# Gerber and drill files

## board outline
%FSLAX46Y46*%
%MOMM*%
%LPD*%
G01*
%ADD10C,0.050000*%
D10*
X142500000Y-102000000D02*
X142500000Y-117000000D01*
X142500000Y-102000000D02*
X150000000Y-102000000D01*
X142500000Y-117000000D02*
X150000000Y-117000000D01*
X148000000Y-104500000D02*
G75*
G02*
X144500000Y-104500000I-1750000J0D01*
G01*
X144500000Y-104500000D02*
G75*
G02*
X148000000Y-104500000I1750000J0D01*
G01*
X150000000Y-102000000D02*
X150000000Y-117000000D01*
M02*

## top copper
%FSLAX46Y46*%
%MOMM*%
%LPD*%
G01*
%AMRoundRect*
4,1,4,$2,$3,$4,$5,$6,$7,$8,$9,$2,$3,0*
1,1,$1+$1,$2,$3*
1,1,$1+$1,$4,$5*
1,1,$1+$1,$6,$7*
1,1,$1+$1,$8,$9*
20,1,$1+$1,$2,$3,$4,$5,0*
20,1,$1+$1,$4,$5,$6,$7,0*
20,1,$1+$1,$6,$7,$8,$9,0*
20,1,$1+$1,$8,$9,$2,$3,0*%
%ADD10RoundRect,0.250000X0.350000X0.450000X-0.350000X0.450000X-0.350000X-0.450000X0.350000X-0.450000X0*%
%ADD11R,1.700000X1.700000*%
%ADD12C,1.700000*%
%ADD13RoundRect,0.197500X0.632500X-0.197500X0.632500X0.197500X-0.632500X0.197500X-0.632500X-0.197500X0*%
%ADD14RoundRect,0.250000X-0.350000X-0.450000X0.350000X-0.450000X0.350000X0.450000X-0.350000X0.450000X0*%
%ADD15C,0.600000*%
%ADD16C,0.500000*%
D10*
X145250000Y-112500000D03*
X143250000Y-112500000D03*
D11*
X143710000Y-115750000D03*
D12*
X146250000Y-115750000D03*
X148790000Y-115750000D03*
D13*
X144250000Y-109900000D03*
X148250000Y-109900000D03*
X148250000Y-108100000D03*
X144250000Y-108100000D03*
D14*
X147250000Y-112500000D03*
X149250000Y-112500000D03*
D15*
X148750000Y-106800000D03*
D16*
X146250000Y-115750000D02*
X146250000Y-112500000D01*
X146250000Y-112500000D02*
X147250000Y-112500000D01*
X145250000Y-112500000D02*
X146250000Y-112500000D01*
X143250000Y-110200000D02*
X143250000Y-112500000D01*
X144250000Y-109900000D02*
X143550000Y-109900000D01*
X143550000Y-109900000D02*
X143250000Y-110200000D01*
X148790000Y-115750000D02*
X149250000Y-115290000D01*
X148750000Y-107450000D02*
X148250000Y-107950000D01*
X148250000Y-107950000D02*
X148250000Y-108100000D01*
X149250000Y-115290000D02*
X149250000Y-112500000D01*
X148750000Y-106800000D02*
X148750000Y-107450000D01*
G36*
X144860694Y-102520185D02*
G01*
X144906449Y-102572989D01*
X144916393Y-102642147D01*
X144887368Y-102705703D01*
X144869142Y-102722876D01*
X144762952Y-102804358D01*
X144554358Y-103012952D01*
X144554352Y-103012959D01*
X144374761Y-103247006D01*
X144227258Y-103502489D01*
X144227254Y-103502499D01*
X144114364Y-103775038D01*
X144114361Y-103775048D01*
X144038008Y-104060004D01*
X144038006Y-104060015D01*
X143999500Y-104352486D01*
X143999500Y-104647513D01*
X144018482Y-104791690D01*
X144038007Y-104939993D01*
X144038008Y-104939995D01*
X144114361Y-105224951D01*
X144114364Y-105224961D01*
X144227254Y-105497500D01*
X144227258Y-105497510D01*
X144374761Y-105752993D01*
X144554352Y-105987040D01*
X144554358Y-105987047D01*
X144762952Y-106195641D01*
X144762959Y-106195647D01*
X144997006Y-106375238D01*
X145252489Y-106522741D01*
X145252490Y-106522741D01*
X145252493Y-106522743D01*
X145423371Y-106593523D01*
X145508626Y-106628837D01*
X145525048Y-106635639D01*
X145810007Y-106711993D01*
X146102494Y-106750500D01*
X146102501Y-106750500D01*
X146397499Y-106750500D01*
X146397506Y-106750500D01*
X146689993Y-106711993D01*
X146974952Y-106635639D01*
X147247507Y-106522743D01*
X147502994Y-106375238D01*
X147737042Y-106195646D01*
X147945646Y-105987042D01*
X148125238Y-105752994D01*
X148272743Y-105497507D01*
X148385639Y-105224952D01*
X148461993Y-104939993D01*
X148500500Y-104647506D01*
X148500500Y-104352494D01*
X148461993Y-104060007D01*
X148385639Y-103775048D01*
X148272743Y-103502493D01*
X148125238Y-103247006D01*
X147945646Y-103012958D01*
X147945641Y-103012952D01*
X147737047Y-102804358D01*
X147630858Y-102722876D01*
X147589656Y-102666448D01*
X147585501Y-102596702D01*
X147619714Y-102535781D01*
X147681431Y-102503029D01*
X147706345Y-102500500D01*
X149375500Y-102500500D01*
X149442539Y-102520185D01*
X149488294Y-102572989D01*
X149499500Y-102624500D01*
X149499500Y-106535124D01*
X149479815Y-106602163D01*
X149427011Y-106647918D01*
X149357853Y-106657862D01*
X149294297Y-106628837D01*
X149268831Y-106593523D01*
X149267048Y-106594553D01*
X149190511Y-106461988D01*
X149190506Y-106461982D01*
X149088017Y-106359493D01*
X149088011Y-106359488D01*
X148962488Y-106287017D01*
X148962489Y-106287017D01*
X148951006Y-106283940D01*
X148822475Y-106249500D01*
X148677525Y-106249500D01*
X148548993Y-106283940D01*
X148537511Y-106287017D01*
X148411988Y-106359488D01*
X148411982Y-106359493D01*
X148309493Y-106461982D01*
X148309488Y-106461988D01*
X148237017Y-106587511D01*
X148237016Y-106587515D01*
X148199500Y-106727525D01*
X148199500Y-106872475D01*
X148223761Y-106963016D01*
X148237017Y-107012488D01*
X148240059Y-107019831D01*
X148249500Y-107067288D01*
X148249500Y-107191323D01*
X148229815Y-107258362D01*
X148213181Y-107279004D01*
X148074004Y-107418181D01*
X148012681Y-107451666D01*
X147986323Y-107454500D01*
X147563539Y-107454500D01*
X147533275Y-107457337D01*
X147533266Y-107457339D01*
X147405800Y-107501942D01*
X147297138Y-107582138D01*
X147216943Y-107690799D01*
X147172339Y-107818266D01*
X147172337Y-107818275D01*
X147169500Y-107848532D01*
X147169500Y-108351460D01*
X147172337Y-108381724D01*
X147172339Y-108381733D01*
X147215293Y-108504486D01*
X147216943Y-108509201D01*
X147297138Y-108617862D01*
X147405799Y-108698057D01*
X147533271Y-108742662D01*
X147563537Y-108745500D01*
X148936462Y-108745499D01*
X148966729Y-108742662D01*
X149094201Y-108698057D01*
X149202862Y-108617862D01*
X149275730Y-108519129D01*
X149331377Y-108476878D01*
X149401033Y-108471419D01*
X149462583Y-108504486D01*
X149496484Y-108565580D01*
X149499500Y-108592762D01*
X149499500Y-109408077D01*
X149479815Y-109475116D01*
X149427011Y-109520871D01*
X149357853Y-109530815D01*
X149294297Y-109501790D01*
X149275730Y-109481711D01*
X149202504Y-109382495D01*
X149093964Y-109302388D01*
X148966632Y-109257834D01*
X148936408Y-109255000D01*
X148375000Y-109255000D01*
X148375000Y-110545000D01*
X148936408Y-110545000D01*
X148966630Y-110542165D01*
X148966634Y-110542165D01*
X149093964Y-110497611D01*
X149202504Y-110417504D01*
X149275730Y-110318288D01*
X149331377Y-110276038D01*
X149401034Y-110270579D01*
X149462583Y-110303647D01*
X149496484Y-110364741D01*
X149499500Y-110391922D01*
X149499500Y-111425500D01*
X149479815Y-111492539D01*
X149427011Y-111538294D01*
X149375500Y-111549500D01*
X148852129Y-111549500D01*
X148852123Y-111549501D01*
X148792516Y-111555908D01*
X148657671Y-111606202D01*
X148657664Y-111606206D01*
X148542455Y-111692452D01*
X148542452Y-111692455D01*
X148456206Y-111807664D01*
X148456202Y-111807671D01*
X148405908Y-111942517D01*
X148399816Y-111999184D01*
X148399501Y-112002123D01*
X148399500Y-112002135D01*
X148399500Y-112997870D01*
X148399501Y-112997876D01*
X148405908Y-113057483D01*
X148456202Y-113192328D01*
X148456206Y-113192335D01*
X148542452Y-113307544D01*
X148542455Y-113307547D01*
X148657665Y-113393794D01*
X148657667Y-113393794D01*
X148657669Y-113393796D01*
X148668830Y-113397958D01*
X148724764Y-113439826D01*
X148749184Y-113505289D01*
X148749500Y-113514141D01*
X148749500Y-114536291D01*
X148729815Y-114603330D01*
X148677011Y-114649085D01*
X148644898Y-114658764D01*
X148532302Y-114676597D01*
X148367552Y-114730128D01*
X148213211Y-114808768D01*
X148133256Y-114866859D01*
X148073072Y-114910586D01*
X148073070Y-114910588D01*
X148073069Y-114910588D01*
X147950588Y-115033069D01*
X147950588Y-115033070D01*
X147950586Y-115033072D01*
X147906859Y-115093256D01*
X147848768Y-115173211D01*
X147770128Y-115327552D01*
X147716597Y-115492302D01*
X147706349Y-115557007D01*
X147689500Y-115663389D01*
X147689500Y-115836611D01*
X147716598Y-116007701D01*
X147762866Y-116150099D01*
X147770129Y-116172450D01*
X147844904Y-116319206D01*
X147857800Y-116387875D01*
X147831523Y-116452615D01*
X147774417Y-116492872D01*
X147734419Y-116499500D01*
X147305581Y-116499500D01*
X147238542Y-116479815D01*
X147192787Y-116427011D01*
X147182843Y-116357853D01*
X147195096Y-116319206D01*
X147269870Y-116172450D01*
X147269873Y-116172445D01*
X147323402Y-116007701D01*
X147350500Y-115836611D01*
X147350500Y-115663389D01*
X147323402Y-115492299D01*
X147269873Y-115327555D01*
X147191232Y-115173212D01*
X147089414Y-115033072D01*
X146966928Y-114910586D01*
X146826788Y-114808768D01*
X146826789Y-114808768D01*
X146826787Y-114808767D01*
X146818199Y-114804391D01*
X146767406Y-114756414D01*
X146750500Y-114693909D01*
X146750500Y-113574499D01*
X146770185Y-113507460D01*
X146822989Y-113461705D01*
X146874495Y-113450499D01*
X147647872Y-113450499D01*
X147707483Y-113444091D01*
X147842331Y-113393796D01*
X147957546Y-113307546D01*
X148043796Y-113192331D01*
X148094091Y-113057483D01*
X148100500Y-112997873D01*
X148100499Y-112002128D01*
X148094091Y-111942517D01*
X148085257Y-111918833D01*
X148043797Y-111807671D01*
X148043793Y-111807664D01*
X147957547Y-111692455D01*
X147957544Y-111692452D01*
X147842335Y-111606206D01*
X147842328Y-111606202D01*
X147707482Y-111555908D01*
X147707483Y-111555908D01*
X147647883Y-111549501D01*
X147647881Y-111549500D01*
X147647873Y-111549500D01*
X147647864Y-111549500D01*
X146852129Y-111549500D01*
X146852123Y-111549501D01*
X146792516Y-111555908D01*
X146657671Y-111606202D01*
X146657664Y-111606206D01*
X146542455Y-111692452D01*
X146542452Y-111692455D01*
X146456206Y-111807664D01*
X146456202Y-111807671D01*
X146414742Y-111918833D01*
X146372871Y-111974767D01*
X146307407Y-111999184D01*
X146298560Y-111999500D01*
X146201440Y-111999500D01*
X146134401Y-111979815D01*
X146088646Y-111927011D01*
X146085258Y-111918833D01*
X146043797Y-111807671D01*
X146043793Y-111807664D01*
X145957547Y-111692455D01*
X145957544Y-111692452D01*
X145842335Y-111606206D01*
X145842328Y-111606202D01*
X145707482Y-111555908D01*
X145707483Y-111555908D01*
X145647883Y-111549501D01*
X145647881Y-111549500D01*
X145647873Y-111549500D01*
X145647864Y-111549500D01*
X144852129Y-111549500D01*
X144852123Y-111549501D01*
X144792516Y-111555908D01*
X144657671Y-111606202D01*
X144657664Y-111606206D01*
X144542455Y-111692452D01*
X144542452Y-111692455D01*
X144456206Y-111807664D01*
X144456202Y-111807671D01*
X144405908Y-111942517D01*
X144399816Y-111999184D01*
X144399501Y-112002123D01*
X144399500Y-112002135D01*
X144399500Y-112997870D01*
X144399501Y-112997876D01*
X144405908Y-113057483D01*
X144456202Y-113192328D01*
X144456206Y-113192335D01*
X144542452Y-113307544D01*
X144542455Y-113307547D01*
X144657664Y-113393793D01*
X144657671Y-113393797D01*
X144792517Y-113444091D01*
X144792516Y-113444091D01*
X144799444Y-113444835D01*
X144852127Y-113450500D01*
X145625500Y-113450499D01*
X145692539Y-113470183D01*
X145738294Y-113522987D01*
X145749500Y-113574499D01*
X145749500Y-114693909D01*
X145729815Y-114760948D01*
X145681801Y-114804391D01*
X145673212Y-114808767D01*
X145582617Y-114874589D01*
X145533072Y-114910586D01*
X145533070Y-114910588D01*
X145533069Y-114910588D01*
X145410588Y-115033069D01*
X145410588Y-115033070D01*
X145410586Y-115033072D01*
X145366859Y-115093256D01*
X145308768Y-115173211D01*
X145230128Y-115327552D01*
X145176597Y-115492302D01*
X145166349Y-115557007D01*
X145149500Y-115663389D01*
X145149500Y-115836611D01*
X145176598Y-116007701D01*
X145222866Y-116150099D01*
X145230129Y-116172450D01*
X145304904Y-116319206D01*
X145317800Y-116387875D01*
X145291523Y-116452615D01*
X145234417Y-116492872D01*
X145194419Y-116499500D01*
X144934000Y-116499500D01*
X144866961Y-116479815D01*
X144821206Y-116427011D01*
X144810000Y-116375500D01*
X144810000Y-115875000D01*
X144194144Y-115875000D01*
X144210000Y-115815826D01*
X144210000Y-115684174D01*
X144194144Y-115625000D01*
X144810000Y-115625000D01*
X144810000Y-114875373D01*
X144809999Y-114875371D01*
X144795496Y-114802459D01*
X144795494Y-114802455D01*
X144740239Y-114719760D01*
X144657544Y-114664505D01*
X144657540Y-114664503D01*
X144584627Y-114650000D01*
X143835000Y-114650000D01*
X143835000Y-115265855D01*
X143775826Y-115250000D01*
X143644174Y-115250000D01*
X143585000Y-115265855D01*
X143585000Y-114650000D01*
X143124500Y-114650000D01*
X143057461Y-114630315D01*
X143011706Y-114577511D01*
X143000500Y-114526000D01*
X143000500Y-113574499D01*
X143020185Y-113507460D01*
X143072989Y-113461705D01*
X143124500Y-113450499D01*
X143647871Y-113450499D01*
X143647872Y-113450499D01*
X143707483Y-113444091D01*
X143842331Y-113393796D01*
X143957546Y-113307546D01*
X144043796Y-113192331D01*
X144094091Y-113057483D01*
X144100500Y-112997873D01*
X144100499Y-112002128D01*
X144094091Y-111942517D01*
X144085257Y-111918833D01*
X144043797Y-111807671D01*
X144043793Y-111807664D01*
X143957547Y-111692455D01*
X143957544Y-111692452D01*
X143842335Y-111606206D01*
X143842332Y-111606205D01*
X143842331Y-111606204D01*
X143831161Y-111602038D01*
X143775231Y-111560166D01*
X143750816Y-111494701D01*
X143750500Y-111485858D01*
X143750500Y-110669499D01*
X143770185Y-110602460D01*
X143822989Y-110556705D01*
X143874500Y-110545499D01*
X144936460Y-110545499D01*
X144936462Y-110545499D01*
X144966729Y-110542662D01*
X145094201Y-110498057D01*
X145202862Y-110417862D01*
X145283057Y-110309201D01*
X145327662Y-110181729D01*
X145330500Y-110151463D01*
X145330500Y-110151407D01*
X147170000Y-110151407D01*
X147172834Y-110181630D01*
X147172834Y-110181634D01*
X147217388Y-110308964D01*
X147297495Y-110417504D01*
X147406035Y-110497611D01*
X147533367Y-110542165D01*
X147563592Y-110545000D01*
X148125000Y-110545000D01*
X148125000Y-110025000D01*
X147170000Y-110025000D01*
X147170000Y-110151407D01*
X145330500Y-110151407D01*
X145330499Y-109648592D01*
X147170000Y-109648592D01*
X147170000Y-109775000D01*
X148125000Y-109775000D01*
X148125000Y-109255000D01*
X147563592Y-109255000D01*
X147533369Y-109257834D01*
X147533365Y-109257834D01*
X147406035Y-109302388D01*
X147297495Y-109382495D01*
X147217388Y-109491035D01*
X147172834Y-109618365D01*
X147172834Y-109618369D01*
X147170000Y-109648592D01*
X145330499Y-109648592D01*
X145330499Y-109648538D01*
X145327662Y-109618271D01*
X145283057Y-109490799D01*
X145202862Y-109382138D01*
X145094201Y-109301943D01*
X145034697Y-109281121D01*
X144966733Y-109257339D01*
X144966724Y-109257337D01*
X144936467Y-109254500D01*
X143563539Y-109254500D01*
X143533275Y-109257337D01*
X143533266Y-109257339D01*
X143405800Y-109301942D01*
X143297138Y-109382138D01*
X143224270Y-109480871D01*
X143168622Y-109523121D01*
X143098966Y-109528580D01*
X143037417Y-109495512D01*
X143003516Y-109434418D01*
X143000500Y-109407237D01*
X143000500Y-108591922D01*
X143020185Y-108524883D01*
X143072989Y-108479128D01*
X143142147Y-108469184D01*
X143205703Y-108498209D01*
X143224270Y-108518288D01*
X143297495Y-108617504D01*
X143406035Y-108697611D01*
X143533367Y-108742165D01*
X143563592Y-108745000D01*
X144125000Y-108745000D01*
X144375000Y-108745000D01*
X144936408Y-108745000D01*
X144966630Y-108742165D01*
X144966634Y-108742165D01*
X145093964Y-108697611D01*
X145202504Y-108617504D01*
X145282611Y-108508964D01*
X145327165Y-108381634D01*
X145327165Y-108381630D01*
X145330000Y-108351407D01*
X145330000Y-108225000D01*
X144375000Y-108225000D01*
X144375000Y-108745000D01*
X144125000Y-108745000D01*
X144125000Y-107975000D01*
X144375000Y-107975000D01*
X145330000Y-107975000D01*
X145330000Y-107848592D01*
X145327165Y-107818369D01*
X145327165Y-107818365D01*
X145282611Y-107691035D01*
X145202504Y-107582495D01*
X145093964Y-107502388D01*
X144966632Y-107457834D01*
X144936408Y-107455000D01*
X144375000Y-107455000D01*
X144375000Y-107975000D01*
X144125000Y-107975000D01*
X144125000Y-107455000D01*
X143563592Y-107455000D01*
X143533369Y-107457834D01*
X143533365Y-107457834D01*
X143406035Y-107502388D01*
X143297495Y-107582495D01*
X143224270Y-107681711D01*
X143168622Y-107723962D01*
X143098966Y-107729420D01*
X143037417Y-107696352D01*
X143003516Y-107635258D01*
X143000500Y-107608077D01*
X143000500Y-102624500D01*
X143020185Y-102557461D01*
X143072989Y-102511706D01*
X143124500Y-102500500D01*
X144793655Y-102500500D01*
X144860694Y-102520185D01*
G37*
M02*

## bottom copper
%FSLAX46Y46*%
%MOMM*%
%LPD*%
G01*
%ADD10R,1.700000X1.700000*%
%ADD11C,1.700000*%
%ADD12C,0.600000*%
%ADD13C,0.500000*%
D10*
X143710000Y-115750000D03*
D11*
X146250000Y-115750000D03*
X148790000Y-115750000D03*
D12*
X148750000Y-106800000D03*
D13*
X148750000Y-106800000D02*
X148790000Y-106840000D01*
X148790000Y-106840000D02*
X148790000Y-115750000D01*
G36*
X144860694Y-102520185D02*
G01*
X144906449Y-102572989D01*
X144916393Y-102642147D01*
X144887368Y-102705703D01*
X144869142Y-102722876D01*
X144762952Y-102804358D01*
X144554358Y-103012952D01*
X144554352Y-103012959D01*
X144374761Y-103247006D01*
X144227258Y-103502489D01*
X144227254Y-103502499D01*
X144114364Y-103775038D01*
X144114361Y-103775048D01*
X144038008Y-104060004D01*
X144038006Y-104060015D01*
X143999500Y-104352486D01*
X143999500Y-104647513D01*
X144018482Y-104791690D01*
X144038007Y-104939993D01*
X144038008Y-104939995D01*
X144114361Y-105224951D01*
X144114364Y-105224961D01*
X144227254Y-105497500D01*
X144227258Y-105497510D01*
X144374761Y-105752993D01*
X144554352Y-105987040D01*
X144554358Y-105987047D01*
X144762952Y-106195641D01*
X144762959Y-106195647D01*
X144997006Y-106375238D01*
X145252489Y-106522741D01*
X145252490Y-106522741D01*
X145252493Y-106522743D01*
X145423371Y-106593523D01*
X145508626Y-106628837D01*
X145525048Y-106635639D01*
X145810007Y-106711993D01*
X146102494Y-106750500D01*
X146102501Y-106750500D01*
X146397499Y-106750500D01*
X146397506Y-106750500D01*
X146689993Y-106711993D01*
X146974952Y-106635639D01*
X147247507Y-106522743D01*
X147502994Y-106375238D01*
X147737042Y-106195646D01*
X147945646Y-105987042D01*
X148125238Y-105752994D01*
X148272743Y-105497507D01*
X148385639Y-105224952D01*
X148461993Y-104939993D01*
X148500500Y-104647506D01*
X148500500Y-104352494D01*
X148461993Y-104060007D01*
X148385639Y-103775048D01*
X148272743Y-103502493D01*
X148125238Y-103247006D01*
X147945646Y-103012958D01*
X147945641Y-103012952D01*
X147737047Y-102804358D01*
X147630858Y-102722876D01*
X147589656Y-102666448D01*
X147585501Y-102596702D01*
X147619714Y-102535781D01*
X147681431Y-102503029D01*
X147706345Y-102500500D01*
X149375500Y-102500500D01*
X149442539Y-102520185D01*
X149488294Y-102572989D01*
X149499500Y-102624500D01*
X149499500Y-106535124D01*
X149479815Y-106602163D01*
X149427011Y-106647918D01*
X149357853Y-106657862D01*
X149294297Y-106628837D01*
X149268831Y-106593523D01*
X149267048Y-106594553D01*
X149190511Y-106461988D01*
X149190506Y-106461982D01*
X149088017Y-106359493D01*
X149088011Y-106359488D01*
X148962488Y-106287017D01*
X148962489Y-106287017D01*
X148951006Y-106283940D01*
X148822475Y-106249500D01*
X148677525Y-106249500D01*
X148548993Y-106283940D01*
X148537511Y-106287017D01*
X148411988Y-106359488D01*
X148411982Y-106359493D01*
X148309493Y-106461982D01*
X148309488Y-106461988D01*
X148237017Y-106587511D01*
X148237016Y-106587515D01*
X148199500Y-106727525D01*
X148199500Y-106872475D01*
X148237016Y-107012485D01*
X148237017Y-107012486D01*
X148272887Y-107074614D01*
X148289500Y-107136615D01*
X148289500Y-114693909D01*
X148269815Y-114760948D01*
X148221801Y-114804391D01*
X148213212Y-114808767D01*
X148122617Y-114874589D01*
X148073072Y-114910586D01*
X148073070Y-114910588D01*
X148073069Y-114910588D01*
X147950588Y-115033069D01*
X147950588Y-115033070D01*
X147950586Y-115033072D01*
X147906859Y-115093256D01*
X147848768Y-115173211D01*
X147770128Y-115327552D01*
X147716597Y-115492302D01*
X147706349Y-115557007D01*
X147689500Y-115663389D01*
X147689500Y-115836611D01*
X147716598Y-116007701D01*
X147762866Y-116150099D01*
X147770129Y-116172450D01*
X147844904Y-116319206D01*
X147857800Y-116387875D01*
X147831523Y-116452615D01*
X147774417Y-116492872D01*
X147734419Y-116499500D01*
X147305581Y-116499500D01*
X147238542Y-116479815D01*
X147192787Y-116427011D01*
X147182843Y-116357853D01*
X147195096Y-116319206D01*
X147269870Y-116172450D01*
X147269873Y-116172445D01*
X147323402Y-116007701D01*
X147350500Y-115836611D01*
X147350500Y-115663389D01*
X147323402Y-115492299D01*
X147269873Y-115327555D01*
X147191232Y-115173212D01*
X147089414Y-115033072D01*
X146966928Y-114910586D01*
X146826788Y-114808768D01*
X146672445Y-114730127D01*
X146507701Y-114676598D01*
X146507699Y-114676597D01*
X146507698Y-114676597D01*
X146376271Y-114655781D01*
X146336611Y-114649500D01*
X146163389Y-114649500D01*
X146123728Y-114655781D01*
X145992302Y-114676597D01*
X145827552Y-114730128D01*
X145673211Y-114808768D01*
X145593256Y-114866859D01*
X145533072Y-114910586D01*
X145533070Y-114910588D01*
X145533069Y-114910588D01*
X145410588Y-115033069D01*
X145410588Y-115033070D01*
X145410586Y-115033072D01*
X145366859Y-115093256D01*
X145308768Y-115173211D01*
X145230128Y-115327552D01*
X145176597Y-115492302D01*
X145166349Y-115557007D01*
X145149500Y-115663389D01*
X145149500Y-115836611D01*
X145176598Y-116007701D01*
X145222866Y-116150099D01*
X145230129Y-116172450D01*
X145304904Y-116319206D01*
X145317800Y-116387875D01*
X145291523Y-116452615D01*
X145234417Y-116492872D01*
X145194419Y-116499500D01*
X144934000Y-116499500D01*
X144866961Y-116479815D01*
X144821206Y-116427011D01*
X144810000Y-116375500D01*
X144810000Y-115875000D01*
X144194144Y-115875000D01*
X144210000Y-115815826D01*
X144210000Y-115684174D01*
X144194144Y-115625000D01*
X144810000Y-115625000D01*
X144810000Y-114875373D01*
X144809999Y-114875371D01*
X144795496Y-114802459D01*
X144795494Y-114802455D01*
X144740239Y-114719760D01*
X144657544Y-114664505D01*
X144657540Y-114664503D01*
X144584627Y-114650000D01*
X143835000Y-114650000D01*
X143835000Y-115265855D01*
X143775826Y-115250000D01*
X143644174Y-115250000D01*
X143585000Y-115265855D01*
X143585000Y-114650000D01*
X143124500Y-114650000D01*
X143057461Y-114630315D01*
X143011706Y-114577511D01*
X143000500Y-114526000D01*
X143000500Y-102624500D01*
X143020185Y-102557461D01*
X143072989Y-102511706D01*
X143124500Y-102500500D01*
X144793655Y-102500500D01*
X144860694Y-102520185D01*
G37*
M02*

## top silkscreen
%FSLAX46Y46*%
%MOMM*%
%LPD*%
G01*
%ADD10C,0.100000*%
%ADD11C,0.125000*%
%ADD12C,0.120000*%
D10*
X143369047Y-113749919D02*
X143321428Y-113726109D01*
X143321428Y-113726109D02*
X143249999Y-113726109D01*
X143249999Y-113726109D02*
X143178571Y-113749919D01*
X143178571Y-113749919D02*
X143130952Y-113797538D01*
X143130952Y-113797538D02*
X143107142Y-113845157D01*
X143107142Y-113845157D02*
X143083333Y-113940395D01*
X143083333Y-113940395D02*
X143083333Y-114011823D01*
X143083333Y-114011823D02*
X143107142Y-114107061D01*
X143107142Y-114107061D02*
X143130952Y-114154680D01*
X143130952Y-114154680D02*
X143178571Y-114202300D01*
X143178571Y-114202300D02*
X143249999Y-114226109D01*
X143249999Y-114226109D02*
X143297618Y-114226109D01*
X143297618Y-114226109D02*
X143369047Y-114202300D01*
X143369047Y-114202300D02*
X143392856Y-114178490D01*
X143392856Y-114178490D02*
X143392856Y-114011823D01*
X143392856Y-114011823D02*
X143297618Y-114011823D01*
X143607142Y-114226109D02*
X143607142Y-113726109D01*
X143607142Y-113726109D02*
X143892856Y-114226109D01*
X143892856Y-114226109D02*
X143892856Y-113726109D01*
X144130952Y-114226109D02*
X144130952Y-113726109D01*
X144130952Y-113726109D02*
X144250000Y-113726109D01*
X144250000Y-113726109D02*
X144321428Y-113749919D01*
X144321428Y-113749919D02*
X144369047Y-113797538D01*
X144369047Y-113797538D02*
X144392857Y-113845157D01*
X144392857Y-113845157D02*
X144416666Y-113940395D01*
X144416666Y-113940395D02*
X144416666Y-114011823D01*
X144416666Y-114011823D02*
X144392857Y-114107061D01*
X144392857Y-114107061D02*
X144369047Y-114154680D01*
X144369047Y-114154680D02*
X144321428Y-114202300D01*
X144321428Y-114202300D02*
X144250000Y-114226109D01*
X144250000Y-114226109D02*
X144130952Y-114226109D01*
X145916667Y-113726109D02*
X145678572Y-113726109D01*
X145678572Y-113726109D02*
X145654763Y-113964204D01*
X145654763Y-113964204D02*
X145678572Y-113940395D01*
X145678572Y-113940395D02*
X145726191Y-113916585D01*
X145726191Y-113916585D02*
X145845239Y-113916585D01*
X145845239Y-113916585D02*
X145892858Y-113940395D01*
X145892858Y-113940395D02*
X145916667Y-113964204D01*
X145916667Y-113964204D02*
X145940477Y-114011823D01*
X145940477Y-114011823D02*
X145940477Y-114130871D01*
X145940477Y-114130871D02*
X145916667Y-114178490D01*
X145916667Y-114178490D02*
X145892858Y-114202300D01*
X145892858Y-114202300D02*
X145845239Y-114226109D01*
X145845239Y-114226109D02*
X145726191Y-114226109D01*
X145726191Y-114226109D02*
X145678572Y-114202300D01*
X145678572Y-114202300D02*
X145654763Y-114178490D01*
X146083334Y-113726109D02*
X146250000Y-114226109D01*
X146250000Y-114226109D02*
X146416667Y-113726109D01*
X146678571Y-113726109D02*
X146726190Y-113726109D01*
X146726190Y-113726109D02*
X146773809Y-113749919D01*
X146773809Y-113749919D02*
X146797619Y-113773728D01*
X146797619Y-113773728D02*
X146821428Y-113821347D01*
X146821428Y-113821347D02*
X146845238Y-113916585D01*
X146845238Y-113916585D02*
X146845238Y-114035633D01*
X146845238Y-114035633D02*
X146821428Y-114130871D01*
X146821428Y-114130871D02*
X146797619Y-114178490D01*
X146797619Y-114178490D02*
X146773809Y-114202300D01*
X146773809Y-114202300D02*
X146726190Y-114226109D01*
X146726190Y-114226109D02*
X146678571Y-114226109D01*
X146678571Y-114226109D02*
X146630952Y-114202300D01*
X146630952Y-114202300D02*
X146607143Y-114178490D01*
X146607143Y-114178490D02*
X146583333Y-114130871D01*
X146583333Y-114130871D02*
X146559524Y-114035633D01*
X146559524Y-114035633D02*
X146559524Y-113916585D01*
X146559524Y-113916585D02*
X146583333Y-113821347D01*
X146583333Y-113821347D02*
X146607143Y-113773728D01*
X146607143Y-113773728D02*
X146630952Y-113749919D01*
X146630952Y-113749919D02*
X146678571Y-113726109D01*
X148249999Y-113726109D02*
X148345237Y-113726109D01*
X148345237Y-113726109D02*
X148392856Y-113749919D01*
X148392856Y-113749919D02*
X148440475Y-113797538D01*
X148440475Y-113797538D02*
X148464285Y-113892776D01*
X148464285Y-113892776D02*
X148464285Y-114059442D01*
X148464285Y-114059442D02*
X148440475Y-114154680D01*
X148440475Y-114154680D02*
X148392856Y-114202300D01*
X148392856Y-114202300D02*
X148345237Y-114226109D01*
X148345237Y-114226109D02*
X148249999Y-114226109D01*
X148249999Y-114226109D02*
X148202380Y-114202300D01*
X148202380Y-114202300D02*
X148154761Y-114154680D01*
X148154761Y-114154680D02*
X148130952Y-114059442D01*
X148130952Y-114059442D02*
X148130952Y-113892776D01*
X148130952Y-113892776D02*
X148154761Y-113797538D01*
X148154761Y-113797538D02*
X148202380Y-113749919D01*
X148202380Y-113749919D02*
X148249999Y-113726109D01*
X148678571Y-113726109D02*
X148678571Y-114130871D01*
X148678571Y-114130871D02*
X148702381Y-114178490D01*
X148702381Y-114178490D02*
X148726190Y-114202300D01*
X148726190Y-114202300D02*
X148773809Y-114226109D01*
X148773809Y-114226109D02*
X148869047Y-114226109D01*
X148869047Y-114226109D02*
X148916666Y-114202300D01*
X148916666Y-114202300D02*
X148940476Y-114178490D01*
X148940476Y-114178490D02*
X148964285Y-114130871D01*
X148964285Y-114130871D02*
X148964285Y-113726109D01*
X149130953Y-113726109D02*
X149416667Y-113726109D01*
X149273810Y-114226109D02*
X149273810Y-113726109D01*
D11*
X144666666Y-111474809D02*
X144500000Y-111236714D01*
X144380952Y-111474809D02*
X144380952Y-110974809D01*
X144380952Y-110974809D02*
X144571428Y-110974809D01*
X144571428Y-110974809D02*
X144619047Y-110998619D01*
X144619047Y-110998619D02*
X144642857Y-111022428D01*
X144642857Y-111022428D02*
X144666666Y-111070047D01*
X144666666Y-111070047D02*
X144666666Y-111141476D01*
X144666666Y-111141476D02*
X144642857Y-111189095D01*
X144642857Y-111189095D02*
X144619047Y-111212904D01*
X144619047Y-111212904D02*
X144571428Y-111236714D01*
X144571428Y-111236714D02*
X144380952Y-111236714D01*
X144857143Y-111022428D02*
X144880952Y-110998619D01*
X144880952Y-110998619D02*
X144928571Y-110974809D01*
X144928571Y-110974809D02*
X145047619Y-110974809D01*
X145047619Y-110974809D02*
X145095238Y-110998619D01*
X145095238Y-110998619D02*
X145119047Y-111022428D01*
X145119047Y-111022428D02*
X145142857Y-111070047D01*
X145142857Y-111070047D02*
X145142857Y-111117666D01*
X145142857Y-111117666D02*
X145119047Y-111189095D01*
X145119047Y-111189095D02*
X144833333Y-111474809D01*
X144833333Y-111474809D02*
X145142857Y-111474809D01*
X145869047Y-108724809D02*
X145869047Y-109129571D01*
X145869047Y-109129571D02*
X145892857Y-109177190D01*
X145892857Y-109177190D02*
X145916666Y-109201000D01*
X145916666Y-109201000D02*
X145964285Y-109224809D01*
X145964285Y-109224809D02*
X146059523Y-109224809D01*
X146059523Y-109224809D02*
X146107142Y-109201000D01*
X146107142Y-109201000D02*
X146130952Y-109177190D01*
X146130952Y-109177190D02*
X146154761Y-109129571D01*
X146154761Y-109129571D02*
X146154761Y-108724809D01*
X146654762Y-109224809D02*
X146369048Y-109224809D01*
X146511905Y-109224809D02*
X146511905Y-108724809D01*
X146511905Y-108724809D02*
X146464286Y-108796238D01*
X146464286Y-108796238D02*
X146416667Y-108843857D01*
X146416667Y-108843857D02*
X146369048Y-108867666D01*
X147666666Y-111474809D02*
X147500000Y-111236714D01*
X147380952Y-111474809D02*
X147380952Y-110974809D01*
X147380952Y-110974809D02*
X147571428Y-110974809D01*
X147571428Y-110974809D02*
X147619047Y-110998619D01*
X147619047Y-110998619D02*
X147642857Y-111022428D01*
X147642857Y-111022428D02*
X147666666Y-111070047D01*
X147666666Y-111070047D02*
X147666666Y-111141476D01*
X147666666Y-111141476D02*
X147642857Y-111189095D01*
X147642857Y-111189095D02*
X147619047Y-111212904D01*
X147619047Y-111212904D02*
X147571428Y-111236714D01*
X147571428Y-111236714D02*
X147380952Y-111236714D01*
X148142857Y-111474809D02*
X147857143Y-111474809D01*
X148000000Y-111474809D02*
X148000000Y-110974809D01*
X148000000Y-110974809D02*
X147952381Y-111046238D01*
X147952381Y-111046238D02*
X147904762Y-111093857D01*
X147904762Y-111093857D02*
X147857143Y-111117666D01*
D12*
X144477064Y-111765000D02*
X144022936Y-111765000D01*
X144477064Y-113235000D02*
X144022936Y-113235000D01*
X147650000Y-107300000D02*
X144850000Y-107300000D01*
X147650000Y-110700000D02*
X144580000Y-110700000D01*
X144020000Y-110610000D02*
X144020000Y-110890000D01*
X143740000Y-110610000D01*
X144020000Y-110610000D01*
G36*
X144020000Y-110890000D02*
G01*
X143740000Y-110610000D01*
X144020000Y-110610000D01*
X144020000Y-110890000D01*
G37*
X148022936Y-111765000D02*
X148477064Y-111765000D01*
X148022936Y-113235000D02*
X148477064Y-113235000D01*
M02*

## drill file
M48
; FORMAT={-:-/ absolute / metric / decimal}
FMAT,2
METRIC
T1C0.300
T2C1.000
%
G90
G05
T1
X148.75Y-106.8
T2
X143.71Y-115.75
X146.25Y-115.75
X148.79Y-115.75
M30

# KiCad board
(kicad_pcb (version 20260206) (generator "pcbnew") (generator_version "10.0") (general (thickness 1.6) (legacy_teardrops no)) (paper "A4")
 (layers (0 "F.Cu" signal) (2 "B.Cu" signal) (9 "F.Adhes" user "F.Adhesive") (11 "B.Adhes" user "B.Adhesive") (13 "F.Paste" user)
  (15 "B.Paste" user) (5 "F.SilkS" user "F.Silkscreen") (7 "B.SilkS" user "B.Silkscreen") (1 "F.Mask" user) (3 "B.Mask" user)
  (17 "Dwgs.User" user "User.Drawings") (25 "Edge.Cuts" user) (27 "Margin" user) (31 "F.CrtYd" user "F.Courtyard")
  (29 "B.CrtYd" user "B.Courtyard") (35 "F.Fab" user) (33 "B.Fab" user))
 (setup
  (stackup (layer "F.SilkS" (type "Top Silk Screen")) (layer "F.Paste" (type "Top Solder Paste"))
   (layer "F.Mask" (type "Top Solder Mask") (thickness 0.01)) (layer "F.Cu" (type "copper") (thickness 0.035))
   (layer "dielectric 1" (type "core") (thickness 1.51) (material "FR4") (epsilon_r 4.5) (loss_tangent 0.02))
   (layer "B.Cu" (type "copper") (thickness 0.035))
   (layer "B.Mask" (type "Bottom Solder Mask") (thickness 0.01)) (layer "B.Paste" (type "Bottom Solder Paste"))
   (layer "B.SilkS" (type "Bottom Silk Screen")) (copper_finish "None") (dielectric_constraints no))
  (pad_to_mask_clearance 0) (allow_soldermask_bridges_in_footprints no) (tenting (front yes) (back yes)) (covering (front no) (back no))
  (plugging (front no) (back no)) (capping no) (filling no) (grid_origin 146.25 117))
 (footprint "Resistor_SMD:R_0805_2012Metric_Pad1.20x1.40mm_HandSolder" (layer "F.Cu") (at 144.25 112.5 180)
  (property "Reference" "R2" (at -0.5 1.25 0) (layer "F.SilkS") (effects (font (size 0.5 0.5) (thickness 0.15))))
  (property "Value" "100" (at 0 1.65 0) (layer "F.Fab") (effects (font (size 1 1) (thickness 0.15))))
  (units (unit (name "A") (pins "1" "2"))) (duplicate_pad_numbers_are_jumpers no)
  (fp_line (start -0.227064 0.735) (end 0.227064 0.735) (stroke (width 0.12) (type solid)) (layer "F.SilkS"))
  (fp_line (start -0.227064 -0.735) (end 0.227064 -0.735) (stroke (width 0.12) (type solid)) (layer "F.SilkS"))
  (pad "1" smd roundrect (at -1 0 180) (size 1.2 1.4) (layers "F.Cu" "F.Mask" "F.Paste") (roundrect_rratio 0.208333) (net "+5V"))
  (pad "2" smd roundrect (at 1 0 180) (size 1.2 1.4) (layers "F.Cu" "F.Mask" "F.Paste") (roundrect_rratio 0.208333) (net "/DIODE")))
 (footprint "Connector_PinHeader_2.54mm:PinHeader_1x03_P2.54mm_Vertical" (layer "F.Cu") (at 143.71 115.75 90)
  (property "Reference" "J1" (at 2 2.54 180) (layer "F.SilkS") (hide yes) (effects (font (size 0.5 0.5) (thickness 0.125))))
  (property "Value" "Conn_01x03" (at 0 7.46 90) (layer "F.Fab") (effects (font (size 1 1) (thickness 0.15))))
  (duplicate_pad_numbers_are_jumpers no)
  (pad "1" thru_hole rect (at 0 0 90) (size 1.7 1.7) (drill 1) (layers "*.Cu" "*.Mask") (remove_unused_layers no) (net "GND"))
  (pad "2" thru_hole circle (at 0 2.54 90) (size 1.7 1.7) (drill 1) (layers "*.Cu" "*.Mask") (remove_unused_layers no) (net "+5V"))
  (pad "3" thru_hole circle (at 0 5.08 90) (size 1.7 1.7) (drill 1) (layers "*.Cu" "*.Mask") (remove_unused_layers no) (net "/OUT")))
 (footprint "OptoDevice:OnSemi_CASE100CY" (layer "F.Cu") (at 146.25 109 90)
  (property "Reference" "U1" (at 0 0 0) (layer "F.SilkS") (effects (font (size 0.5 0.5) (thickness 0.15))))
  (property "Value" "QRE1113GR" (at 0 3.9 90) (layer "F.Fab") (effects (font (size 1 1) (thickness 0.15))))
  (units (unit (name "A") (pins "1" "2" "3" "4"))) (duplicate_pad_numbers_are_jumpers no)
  (fp_line (start 1.7 1.4) (end 1.7 -1.4) (stroke (width 0.12) (type solid)) (layer "F.SilkS"))
  (fp_line (start -1.7 1.4) (end -1.7 -1.67) (stroke (width 0.12) (type solid)) (layer "F.SilkS"))
  (fp_poly
   (pts (xy -1.61 -2.23) (xy -1.89 -2.23) (xy -1.61 -2.51) (xy -1.61 -2.23)) (stroke (width 0.12) (type solid)) (fill yes) (layer "F.SilkS"))
  (pad "1" smd roundrect (at -0.9 -2 90) (size 0.79 1.66) (layers "F.Cu" "F.Mask" "F.Paste") (roundrect_rratio 0.25) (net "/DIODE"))
  (pad "2" smd roundrect (at -0.9 2 90) (size 0.79 1.66) (layers "F.Cu" "F.Mask" "F.Paste") (roundrect_rratio 0.25) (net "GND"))
  (pad "3" smd roundrect (at 0.9 2 90) (size 0.79 1.66) (layers "F.Cu" "F.Mask" "F.Paste") (roundrect_rratio 0.25) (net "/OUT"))
  (pad "4" smd roundrect (at 0.9 -2 90) (size 0.79 1.66) (layers "F.Cu" "F.Mask" "F.Paste") (roundrect_rratio 0.25) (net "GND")))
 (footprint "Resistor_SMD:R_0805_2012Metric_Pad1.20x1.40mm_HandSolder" (layer "F.Cu") (at 148.25 112.5)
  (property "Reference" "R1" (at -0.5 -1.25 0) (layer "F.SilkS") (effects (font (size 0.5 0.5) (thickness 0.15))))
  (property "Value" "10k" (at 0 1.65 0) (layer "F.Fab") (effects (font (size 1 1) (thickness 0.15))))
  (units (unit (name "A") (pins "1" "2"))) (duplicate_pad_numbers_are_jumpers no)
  (fp_line (start -0.227064 -0.735) (end 0.227064 -0.735) (stroke (width 0.12) (type solid)) (layer "F.SilkS"))
  (fp_line (start -0.227064 0.735) (end 0.227064 0.735) (stroke (width 0.12) (type solid)) (layer "F.SilkS"))
  (pad "1" smd roundrect (at -1 0) (size 1.2 1.4) (layers "F.Cu" "F.Mask" "F.Paste") (roundrect_rratio 0.208333) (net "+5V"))
  (pad "2" smd roundrect (at 1 0) (size 1.2 1.4) (layers "F.Cu" "F.Mask" "F.Paste") (roundrect_rratio 0.208333) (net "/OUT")))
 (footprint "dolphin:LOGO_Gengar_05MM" (layer "B.Cu") (at 146.25 109 180)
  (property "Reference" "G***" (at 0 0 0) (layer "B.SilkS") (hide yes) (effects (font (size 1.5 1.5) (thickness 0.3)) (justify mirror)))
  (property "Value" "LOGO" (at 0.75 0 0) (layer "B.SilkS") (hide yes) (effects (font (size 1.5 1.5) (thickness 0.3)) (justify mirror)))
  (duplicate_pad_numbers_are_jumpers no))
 (gr_line (start 142.5 102) (end 142.5 117) (stroke (width 0.05) (type default)) (layer "Edge.Cuts"))
 (gr_line (start 142.5 102) (end 150 102) (stroke (width 0.05) (type default)) (layer "Edge.Cuts"))
 (gr_line (start 142.5 117) (end 150 117) (stroke (width 0.05) (type default)) (layer "Edge.Cuts"))
 (gr_circle (center 146.25 104.5) (end 148 104.5) (stroke (width 0.05) (type default)) (fill no) (layer "Edge.Cuts"))
 (gr_line (start 150 102) (end 150 117) (stroke (width 0.05) (type default)) (layer "Edge.Cuts"))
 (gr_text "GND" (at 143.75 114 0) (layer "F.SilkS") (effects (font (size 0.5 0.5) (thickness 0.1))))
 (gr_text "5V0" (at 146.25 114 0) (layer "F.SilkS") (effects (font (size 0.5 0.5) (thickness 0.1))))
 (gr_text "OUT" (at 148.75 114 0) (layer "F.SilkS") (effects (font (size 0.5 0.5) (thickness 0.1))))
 (segment (start 146.25 115.75) (end 146.25 112.5) (width 0.5) (layer "F.Cu") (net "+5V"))
 (segment (start 146.25 112.5) (end 147.25 112.5) (width 0.5) (layer "F.Cu") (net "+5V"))
 (segment (start 145.25 112.5) (end 146.25 112.5) (width 0.5) (layer "F.Cu") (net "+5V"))
 (segment (start 143.25 110.2) (end 143.25 112.5) (width 0.5) (layer "F.Cu") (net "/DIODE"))
 (segment (start 144.25 109.9) (end 143.55 109.9) (width 0.5) (layer "F.Cu") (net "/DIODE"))
 (segment (start 143.55 109.9) (end 143.25 110.2) (width 0.5) (layer "F.Cu") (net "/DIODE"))
 (segment (start 148.79 115.75) (end 149.25 115.29) (width 0.5) (layer "F.Cu") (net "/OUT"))
 (segment (start 148.75 107.45) (end 148.25 107.95) (width 0.5) (layer "F.Cu") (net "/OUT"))
 (segment (start 148.25 107.95) (end 148.25 108.1) (width 0.5) (layer "F.Cu") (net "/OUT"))
 (segment (start 149.25 115.29) (end 149.25 112.5) (width 0.5) (layer "F.Cu") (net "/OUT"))
 (segment (start 148.75 106.8) (end 148.75 107.45) (width 0.5) (layer "F.Cu") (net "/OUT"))
 (via (at 148.75 106.8) (size 0.6) (drill 0.3) (layers "F.Cu" "B.Cu") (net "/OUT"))
 (segment (start 148.75 106.8) (end 148.79 106.84) (width 0.5) (layer "B.Cu") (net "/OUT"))
 (segment (start 148.79 106.84) (end 148.79 115.75) (width 0.5) (layer "B.Cu") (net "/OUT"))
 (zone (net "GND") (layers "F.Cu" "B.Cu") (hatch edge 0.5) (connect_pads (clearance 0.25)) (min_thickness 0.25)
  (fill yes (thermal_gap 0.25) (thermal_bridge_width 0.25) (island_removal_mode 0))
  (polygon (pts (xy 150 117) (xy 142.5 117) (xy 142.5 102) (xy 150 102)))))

